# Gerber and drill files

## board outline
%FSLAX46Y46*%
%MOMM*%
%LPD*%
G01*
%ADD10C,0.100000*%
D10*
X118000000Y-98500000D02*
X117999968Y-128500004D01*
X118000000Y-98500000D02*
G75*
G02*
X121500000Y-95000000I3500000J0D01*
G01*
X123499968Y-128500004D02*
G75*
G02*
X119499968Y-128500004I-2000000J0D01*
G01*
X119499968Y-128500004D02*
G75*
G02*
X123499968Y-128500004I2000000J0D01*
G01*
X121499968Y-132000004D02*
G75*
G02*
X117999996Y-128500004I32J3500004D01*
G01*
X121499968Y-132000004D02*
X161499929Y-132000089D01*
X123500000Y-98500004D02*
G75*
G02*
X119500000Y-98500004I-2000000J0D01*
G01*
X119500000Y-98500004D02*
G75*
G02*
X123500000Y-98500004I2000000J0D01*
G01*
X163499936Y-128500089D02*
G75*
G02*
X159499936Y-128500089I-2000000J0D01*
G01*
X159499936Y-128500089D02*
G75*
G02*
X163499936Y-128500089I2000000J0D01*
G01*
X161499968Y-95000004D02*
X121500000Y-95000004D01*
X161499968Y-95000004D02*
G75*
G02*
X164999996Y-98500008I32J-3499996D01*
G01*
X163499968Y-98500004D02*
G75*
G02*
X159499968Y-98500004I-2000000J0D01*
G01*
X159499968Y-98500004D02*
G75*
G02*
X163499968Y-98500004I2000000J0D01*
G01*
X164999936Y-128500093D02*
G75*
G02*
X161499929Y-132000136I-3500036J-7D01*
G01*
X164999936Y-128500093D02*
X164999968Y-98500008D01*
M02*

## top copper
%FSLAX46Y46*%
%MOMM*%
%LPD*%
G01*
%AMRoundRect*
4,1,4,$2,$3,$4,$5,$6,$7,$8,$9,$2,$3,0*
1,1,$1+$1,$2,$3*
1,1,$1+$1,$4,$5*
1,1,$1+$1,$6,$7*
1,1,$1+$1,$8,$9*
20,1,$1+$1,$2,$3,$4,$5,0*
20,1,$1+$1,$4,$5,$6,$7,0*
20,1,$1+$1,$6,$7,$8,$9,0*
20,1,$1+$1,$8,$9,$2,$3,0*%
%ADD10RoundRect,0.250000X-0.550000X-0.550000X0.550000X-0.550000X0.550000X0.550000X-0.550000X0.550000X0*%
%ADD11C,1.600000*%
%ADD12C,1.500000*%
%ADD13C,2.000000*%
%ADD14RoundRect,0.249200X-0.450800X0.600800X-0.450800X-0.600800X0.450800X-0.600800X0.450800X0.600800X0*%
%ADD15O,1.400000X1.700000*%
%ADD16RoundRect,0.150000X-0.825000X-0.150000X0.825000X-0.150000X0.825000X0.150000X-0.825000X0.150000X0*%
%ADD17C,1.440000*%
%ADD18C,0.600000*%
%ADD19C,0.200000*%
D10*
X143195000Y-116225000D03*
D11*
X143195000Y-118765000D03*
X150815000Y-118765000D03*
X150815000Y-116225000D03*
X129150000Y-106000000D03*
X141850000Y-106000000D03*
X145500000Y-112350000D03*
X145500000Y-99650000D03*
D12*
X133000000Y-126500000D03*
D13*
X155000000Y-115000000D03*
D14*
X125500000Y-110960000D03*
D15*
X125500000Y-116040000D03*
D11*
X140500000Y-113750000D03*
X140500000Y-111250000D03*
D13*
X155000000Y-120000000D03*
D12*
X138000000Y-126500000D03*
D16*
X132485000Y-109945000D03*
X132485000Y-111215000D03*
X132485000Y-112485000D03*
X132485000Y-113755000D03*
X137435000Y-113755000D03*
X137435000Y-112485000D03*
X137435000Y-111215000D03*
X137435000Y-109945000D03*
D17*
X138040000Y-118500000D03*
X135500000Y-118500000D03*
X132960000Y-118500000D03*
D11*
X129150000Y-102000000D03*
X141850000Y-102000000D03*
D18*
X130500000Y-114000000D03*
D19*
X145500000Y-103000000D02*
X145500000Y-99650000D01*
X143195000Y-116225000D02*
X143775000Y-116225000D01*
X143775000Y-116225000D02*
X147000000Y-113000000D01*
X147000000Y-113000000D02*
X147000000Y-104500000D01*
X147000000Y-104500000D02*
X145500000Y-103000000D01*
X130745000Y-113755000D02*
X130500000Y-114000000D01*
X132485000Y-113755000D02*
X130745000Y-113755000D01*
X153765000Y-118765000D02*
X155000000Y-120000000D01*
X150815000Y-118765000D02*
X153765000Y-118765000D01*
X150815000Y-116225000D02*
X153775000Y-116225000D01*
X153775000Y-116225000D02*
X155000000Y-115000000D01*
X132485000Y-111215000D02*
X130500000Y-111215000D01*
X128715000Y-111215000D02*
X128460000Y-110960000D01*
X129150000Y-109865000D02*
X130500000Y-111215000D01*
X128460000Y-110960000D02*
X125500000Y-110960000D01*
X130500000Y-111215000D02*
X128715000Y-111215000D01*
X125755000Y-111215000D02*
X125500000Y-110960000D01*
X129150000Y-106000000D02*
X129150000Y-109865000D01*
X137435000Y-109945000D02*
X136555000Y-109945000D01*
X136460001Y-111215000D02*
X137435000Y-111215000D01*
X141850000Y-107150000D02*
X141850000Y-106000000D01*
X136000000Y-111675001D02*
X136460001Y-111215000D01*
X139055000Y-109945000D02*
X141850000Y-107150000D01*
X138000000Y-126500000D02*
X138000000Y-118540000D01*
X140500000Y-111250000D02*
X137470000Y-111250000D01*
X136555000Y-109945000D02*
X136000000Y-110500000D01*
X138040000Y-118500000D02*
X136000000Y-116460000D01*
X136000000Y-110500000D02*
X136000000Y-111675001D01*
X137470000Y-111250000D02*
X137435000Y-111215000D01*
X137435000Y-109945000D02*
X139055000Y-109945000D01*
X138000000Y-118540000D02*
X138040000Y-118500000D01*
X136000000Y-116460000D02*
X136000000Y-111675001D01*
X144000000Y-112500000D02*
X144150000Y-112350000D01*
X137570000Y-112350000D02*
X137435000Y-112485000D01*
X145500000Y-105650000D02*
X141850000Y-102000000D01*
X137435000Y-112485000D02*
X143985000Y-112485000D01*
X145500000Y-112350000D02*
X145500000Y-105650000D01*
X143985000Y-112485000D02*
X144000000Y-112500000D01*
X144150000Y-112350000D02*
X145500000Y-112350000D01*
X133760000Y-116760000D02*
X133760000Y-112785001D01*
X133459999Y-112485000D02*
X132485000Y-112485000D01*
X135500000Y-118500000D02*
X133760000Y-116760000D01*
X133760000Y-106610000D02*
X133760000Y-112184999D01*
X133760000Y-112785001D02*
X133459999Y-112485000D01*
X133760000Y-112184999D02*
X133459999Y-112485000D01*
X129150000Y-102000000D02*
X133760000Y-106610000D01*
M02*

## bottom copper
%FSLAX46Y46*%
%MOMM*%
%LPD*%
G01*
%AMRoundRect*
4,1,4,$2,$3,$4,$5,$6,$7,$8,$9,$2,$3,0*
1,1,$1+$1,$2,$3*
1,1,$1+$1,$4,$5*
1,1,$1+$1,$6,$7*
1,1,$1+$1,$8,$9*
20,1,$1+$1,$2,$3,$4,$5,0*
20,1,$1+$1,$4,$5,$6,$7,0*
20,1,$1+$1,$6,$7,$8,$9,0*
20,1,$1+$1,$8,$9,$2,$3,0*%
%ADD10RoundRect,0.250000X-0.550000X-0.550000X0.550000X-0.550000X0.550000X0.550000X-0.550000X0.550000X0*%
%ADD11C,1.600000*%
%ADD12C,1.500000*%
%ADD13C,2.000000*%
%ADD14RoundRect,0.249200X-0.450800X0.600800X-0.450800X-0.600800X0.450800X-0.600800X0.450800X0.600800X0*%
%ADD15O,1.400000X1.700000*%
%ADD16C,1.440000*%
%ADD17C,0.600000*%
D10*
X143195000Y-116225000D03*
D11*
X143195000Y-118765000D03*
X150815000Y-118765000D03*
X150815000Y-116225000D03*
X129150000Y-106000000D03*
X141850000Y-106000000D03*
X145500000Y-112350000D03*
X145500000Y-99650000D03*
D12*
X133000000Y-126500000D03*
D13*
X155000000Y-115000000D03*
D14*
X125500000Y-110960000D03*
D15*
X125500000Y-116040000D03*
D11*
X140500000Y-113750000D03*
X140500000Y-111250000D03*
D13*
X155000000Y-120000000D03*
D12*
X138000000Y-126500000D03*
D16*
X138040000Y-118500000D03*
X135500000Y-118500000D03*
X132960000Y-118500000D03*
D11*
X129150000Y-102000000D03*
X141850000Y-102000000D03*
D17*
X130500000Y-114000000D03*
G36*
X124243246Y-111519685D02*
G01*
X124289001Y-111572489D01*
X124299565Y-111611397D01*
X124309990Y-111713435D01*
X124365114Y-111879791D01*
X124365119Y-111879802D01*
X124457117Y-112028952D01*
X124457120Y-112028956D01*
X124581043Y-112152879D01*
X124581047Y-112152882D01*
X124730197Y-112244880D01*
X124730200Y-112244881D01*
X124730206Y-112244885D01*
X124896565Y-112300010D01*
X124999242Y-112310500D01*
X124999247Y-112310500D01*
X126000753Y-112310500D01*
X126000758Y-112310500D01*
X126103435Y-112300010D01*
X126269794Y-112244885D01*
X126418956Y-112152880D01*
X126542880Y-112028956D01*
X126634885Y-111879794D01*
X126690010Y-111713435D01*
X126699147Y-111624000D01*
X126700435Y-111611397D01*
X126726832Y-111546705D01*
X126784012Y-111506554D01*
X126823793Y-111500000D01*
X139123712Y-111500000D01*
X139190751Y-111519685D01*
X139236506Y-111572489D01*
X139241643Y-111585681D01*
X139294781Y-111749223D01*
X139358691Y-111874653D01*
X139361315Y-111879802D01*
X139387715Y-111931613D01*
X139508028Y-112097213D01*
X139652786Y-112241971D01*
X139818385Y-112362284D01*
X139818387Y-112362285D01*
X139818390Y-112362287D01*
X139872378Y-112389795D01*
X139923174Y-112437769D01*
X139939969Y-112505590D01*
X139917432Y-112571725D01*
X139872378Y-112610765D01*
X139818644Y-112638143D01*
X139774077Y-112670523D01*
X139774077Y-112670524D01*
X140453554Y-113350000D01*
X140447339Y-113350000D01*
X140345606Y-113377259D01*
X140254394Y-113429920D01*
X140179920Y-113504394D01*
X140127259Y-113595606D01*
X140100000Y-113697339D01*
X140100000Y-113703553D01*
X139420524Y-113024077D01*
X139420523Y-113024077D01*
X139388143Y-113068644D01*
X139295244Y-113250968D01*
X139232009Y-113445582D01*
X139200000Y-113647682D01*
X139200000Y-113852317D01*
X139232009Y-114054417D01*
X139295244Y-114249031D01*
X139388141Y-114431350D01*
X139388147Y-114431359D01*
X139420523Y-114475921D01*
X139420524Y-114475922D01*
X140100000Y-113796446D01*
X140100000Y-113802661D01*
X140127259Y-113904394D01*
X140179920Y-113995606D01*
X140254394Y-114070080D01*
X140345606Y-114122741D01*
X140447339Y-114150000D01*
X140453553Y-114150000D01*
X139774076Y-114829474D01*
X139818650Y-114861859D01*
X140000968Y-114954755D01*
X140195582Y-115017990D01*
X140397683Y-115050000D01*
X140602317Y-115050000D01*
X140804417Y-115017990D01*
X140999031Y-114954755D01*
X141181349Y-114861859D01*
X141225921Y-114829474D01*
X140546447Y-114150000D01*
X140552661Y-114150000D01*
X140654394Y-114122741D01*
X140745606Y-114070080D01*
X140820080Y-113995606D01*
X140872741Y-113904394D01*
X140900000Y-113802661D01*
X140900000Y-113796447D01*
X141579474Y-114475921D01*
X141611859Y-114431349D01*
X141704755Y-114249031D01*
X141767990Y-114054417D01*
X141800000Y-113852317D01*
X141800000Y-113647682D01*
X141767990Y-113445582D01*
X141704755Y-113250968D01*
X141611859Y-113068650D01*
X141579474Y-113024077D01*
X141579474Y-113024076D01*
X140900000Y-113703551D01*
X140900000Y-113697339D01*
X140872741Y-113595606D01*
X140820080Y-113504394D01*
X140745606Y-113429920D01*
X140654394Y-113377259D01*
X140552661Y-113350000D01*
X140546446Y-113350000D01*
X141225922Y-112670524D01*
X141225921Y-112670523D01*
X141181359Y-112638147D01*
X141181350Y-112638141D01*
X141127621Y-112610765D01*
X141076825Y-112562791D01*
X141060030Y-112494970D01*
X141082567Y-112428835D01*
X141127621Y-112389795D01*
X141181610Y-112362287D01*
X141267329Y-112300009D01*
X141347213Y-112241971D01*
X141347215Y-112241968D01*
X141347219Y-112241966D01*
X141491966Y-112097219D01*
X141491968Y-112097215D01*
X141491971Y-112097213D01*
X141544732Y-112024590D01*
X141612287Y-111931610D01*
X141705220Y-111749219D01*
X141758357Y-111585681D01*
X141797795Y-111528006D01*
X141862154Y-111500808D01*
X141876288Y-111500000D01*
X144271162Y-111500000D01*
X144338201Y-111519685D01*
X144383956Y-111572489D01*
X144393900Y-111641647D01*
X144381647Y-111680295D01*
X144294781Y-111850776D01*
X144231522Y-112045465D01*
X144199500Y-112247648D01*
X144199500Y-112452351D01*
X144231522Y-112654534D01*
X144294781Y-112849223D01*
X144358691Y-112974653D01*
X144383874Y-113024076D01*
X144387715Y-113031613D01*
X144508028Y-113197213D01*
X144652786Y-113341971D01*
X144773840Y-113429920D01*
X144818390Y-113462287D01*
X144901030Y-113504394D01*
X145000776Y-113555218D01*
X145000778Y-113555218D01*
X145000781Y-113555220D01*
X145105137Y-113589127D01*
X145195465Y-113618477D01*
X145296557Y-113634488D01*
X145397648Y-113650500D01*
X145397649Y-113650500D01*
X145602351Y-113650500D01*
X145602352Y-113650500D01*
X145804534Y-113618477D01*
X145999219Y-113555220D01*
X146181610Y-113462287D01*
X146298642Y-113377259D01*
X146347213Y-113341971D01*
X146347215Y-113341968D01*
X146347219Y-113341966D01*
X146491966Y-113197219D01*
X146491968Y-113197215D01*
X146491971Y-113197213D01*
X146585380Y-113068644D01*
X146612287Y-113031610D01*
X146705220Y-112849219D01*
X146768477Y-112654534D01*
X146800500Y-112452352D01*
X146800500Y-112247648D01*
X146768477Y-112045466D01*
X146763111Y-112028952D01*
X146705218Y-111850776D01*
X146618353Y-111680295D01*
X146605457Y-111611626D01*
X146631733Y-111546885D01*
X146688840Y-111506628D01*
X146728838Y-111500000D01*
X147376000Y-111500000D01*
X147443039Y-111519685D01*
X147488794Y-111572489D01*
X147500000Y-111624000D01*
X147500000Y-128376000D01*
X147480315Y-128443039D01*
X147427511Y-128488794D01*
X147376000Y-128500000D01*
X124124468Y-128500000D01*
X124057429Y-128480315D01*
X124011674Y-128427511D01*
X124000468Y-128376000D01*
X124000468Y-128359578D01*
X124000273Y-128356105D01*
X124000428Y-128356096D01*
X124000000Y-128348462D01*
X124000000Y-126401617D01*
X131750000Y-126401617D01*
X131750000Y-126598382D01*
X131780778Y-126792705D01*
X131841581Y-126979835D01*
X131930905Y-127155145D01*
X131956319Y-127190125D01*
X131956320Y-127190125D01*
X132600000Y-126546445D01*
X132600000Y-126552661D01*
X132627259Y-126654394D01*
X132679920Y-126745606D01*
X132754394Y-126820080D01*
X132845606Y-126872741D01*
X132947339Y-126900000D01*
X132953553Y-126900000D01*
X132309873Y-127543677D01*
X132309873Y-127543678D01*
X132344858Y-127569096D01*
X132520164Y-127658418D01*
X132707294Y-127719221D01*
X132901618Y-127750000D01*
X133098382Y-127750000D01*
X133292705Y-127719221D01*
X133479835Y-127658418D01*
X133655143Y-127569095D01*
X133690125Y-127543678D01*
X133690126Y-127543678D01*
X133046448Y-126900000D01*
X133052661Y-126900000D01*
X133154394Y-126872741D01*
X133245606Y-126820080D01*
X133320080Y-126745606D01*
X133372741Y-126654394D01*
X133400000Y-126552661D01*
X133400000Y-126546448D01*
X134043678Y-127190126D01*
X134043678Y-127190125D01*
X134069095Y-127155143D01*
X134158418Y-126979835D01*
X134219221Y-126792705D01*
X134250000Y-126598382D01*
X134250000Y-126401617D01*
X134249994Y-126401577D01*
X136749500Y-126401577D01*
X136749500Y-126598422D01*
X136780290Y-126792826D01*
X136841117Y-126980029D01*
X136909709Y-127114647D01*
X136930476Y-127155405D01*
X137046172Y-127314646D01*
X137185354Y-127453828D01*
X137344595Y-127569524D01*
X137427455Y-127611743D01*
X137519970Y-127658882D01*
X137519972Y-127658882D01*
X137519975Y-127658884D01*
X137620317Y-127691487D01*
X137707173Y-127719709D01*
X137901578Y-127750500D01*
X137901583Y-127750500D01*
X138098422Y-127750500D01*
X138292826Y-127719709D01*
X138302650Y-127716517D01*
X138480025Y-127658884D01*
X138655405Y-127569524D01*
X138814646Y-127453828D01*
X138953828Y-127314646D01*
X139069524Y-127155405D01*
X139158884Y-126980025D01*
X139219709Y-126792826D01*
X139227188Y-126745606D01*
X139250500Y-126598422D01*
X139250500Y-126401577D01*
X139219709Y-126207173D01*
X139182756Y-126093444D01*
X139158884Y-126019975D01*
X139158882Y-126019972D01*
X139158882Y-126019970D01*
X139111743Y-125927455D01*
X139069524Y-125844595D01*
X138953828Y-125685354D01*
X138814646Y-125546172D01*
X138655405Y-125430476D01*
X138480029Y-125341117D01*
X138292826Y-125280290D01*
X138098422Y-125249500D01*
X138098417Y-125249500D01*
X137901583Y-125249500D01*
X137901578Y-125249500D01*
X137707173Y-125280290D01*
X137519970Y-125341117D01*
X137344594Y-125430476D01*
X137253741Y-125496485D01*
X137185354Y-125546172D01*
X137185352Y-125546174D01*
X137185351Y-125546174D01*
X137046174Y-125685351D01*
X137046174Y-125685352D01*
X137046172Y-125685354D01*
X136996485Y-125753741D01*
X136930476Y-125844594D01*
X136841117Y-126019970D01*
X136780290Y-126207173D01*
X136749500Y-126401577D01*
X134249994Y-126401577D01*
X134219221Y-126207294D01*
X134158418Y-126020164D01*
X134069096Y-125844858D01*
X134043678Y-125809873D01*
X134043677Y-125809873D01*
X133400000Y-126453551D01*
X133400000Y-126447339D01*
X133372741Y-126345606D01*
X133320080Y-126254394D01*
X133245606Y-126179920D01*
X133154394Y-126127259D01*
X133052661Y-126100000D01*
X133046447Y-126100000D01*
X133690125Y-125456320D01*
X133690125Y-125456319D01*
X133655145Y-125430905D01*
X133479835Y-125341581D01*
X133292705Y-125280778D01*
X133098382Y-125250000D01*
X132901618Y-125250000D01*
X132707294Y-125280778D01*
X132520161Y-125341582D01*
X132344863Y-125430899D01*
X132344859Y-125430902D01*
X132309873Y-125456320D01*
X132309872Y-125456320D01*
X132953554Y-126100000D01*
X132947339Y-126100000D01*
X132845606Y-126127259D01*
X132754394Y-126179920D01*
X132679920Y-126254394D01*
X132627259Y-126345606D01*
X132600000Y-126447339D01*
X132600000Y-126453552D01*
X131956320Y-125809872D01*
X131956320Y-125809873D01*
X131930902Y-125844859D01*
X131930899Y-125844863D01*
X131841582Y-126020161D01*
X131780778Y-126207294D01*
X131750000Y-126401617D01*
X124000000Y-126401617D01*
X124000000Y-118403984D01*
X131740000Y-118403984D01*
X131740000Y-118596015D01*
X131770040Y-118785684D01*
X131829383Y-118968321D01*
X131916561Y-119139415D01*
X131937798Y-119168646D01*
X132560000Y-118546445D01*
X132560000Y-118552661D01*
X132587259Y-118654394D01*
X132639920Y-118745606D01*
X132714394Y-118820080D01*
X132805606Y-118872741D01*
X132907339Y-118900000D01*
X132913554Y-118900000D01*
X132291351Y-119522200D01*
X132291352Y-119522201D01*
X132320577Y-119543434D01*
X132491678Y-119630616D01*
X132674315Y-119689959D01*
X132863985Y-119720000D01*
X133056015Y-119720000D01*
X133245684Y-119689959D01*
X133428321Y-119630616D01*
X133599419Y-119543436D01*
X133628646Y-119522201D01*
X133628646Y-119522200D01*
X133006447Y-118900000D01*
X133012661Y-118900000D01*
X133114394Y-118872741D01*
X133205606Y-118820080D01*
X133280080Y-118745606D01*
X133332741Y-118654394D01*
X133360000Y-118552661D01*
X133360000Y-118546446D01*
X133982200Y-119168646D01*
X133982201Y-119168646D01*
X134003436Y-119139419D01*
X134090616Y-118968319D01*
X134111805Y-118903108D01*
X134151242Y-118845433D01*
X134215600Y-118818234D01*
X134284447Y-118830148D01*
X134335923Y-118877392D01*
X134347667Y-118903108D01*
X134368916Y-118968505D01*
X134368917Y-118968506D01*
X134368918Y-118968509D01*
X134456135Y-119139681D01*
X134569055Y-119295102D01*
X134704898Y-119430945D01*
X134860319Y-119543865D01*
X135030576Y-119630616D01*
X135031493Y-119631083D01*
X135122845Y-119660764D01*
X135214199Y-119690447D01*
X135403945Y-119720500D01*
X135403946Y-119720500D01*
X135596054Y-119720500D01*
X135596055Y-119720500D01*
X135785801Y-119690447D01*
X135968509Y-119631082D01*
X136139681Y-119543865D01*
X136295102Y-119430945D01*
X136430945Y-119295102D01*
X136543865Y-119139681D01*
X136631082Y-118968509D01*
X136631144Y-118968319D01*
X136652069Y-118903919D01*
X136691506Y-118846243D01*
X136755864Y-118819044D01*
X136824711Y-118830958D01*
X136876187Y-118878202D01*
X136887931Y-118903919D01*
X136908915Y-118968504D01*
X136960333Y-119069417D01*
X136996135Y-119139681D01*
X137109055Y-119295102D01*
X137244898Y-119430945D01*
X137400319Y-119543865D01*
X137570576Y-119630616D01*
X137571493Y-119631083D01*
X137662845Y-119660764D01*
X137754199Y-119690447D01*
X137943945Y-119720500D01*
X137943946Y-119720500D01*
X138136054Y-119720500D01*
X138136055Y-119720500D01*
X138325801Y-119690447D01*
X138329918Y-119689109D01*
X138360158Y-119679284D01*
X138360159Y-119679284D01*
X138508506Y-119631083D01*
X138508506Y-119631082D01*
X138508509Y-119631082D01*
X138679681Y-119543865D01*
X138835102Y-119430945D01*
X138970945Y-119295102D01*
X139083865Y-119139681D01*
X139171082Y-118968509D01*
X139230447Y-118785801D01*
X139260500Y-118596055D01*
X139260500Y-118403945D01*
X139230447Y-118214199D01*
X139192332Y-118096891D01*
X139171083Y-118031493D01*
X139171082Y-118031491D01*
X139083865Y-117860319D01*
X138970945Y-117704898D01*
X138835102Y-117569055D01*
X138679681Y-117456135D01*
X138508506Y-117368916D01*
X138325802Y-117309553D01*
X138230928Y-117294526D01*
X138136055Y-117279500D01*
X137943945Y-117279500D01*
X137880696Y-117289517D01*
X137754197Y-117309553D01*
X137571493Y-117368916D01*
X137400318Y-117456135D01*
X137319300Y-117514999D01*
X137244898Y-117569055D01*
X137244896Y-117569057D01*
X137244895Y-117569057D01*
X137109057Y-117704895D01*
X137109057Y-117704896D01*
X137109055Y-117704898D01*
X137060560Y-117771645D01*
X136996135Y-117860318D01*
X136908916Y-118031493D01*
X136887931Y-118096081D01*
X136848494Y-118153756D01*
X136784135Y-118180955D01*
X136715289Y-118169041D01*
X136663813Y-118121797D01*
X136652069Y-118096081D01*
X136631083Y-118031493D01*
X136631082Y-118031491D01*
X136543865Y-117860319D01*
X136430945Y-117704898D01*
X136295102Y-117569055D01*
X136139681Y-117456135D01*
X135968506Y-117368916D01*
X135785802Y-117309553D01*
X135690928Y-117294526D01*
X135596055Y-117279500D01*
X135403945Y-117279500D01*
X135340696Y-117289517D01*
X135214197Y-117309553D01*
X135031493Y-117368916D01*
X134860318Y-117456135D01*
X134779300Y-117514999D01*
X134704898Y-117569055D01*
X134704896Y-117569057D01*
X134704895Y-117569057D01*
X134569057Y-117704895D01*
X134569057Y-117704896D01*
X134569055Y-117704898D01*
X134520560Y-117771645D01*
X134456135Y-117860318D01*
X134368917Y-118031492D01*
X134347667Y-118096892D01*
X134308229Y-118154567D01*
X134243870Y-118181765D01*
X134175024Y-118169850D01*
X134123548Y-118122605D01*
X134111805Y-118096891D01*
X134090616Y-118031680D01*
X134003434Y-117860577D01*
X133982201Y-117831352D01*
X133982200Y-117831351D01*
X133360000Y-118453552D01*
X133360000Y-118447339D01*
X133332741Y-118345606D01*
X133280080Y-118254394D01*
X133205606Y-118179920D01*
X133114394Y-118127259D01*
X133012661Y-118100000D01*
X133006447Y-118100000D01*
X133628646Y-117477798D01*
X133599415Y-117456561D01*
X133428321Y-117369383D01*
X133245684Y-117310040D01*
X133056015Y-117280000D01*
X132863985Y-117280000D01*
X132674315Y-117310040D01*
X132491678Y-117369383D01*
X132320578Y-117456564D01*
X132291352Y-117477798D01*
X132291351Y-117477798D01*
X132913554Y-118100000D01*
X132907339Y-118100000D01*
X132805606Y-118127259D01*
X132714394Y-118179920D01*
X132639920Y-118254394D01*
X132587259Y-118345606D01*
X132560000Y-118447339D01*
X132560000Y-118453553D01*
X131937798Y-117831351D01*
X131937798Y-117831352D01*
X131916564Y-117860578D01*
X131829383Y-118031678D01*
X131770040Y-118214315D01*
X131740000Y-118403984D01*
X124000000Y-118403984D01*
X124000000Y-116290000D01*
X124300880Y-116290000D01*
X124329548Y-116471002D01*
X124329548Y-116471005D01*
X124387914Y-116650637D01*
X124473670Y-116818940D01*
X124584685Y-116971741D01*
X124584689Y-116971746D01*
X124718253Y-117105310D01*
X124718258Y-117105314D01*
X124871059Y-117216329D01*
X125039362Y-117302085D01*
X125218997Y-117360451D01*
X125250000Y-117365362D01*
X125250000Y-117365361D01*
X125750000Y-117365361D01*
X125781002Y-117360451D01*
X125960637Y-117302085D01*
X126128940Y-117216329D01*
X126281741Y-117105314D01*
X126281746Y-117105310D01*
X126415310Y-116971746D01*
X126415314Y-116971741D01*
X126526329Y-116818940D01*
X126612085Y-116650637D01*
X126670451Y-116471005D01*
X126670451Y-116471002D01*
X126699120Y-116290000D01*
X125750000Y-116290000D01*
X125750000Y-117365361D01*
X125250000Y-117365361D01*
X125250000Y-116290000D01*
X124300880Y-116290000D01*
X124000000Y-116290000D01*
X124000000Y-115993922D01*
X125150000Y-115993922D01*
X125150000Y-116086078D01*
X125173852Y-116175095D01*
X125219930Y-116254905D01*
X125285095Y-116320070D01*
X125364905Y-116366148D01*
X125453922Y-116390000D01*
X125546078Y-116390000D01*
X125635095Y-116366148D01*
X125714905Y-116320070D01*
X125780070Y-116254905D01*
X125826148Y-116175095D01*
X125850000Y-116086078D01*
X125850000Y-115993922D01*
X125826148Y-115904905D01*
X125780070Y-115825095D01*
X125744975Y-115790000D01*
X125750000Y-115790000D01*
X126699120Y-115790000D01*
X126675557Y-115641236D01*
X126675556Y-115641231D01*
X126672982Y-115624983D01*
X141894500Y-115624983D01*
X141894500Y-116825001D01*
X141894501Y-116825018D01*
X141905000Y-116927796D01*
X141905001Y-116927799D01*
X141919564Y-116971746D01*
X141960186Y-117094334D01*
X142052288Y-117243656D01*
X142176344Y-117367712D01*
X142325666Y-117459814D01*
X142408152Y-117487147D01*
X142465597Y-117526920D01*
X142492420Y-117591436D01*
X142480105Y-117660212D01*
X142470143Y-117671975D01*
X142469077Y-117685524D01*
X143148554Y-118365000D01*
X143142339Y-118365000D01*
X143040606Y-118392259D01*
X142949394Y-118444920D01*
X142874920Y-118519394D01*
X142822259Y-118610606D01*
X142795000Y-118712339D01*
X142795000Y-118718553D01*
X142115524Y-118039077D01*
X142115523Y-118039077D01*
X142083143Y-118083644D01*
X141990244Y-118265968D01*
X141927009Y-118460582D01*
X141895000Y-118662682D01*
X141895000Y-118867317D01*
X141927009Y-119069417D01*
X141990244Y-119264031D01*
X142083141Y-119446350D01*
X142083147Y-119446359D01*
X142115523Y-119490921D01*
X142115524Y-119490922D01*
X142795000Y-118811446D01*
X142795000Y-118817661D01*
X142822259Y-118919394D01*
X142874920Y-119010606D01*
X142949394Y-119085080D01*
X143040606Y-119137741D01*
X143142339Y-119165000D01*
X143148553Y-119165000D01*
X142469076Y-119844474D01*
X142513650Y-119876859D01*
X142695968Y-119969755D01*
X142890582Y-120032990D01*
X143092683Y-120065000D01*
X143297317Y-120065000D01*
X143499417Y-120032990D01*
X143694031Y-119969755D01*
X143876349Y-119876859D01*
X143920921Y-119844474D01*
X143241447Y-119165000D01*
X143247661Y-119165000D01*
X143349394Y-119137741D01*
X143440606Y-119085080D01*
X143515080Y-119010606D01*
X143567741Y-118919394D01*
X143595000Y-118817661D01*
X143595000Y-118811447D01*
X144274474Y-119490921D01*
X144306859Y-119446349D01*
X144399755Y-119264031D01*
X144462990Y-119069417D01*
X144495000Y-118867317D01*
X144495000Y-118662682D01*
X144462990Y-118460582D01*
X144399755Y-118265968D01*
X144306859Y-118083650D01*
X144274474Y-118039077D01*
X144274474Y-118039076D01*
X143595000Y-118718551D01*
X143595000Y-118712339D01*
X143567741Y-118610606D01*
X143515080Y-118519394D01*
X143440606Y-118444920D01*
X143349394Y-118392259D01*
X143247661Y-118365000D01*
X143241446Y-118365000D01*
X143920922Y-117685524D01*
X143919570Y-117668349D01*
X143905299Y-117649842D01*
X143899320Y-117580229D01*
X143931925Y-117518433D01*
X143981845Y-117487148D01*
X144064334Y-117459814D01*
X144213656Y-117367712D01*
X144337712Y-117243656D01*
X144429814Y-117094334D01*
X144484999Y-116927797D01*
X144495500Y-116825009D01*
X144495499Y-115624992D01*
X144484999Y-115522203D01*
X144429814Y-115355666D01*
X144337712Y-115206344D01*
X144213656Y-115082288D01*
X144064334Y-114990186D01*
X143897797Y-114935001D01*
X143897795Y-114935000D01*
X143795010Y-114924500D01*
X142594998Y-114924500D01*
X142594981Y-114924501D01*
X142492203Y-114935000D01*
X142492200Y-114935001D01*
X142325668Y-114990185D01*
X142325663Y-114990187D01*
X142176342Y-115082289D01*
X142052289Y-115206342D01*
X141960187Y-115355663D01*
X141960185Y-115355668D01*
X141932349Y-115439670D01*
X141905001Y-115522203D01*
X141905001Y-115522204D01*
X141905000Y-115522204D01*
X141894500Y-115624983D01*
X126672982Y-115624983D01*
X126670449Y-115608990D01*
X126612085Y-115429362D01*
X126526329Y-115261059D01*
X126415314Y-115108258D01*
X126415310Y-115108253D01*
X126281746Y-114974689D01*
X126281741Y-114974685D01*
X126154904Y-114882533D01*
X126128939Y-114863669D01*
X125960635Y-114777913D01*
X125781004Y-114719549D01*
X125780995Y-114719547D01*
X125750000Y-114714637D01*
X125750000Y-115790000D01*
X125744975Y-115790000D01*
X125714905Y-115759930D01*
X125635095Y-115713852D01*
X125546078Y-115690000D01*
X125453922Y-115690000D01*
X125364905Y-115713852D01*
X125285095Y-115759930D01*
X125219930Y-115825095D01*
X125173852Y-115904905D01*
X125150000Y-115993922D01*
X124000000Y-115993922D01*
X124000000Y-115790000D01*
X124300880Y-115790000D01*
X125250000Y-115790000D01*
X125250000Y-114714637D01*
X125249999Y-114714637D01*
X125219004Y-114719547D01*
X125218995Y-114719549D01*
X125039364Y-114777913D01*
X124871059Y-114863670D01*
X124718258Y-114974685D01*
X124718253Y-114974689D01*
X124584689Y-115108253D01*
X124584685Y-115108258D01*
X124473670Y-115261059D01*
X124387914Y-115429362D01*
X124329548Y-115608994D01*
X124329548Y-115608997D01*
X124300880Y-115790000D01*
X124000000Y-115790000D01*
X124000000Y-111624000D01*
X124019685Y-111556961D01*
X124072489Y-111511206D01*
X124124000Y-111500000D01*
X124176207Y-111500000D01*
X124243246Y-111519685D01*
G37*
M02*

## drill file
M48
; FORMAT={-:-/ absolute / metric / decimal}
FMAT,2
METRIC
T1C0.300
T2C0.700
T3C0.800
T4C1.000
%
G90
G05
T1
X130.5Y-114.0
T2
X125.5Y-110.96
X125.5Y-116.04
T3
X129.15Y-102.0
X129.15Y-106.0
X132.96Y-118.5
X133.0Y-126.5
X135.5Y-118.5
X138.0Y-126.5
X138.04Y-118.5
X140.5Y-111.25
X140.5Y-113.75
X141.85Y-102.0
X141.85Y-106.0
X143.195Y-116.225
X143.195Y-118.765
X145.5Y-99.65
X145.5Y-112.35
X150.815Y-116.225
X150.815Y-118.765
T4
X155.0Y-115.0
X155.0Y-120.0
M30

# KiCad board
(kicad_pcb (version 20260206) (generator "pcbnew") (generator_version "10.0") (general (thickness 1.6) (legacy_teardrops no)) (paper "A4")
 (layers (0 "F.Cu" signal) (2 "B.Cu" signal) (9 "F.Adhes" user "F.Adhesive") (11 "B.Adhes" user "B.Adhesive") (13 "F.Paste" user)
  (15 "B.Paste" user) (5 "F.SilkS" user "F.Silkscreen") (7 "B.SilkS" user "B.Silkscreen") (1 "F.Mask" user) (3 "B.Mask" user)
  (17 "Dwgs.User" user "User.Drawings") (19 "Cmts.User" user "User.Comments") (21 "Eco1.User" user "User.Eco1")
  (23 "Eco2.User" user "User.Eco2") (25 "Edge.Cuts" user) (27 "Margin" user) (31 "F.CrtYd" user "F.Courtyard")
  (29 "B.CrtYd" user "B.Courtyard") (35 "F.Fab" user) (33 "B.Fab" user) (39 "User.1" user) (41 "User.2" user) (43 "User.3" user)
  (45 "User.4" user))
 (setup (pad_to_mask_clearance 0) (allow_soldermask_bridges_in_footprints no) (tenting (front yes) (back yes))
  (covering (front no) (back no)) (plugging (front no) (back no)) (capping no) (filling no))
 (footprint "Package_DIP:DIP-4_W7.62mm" (layer "F.Cu") (at 143.195 116.225)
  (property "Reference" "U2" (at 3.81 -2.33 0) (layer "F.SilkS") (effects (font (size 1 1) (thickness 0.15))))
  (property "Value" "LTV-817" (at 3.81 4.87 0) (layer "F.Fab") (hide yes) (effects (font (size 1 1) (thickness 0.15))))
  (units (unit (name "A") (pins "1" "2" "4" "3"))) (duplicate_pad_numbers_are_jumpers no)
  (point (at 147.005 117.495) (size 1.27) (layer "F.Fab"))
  (pad "1" thru_hole roundrect (at 0 0) (size 1.6 1.6) (drill 0.8) (layers "*.Cu" "*.Mask") (remove_unused_layers no)
   (roundrect_rratio 0.15625) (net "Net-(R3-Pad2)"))
  (pad "2" thru_hole circle (at 0 2.54) (size 1.6 1.6) (drill 0.8) (layers "*.Cu" "*.Mask") (remove_unused_layers no) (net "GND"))
  (pad "3" thru_hole circle (at 7.62 2.54) (size 1.6 1.6) (drill 0.8) (layers "*.Cu" "*.Mask") (remove_unused_layers no)
   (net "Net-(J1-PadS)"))
  (pad "4" thru_hole circle (at 7.62 0) (size 1.6 1.6) (drill 0.8) (layers "*.Cu" "*.Mask") (remove_unused_layers no) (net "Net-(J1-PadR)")))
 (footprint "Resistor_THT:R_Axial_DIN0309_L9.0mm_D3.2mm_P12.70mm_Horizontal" (layer "F.Cu") (at 129.15 106)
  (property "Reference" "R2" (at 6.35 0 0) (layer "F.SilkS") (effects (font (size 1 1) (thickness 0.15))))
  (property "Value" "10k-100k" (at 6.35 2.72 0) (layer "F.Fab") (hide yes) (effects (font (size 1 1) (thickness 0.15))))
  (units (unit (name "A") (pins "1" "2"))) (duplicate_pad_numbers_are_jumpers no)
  (pad "1" thru_hole circle (at 0 0) (size 1.6 1.6) (drill 0.8) (layers "*.Cu" "*.Mask") (remove_unused_layers no) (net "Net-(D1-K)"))
  (pad "2" thru_hole circle (at 12.7 0) (size 1.6 1.6) (drill 0.8) (layers "*.Cu" "*.Mask") (remove_unused_layers no) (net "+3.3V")))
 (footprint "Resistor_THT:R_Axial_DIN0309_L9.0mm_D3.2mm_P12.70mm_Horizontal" (layer "F.Cu") (at 145.5 112.35 90)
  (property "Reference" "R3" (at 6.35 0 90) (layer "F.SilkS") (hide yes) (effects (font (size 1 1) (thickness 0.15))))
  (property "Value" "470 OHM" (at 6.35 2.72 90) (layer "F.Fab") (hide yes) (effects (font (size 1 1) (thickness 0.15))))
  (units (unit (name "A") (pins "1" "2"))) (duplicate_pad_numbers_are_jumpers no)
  (pad "1" thru_hole circle (at 0 0 90) (size 1.6 1.6) (drill 0.8) (layers "*.Cu" "*.Mask") (remove_unused_layers no) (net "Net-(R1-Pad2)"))
  (pad "2" thru_hole circle (at 12.7 0 90) (size 1.6 1.6) (drill 0.8) (layers "*.Cu" "*.Mask") (remove_unused_layers no)
   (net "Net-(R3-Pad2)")))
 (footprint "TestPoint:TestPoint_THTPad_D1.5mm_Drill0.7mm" (layer "F.Cu") (at 133 126.5 180)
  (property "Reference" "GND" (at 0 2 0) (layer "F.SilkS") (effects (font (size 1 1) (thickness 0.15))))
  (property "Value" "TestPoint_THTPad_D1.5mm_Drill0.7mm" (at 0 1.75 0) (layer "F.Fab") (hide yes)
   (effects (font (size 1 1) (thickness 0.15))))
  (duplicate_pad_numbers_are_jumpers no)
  (pad "1" thru_hole circle (at 0 0 180) (size 1.5 1.5) (drill 0.8) (layers "*.Cu" "*.Mask") (remove_unused_layers no) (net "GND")))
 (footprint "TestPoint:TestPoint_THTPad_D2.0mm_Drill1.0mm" (layer "F.Cu") (at 155 115)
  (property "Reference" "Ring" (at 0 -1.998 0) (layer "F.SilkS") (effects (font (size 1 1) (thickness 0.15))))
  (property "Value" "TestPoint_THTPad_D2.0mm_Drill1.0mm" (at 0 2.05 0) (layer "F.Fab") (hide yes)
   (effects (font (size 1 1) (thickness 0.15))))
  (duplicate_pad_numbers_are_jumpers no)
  (pad "1" thru_hole circle (at 0 0) (size 2 2) (drill 1) (layers "*.Cu" "*.Mask") (remove_unused_layers no) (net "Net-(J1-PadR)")))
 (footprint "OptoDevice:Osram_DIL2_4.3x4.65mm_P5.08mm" (layer "F.Cu") (at 125.5 110.96 -90)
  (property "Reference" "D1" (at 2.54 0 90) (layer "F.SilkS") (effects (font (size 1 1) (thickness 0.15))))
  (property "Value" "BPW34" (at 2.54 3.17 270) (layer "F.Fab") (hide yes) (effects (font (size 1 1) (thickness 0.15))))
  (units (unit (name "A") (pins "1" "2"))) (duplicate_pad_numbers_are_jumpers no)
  (pad "1" thru_hole roundrect (at 0 0 270) (size 1.7 1.4) (drill 0.7) (layers "*.Cu" "*.Mask") (remove_unused_layers no)
   (roundrect_rratio 0.178) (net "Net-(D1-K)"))
  (pad "2" thru_hole oval (at 5.08 0 270) (size 1.7 1.4) (drill 0.7) (layers "*.Cu" "*.Mask") (remove_unused_layers no) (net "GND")))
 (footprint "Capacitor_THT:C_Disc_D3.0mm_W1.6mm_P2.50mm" (layer "F.Cu") (at 140.5 113.75 90)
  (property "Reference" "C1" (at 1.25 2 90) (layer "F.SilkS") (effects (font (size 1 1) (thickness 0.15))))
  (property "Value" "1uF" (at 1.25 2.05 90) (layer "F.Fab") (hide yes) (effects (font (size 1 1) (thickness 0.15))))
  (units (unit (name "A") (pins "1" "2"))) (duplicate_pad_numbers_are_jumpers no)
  (pad "1" thru_hole circle (at 0 0 90) (size 1.6 1.6) (drill 0.8) (layers "*.Cu" "*.Mask") (remove_unused_layers no) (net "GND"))
  (pad "2" thru_hole circle (at 2.5 0 90) (size 1.6 1.6) (drill 0.8) (layers "*.Cu" "*.Mask") (remove_unused_layers no) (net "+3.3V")))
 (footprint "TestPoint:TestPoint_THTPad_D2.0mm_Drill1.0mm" (layer "F.Cu") (at 155 120)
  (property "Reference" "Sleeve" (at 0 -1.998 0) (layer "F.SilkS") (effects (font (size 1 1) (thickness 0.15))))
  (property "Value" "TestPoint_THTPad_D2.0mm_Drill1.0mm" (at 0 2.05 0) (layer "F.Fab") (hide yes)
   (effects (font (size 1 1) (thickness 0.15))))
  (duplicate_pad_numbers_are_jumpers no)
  (pad "1" thru_hole circle (at 0 0) (size 2 2) (drill 1) (layers "*.Cu" "*.Mask") (remove_unused_layers no) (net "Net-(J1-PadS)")))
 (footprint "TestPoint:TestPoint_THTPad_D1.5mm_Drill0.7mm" (layer "F.Cu") (at 138 126.5 180)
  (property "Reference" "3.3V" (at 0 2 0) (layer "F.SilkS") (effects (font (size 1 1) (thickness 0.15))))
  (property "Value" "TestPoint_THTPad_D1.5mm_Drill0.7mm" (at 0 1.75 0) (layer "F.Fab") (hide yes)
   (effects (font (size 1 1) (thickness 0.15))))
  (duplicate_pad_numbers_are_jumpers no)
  (pad "1" thru_hole circle (at 0 0 180) (size 1.5 1.5) (drill 0.8) (layers "*.Cu" "*.Mask") (remove_unused_layers no) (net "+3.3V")))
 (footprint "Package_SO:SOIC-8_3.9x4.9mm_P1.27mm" (layer "F.Cu") (at 134.96 111.85)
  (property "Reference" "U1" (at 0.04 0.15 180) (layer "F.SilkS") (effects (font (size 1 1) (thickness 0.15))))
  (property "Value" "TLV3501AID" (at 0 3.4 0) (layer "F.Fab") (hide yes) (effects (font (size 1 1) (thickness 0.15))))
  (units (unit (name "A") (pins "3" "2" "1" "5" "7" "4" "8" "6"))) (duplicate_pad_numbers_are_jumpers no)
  (pad "1" smd roundrect (at -2.475 -1.905) (size 1.95 0.6) (layers "F.Cu" "F.Mask" "F.Paste") (roundrect_rratio 0.25)
   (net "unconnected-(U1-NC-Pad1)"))
  (pad "2" smd roundrect (at -2.475 -0.635) (size 1.95 0.6) (layers "F.Cu" "F.Mask" "F.Paste") (roundrect_rratio 0.25) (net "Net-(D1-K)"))
  (pad "3" smd roundrect (at -2.475 0.635) (size 1.95 0.6) (layers "F.Cu" "F.Mask" "F.Paste") (roundrect_rratio 0.25) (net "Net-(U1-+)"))
  (pad "4" smd roundrect (at -2.475 1.905) (size 1.95 0.6) (layers "F.Cu" "F.Mask" "F.Paste") (roundrect_rratio 0.25) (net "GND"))
  (pad "5" smd roundrect (at 2.475 1.905) (size 1.95 0.6) (layers "F.Cu" "F.Mask" "F.Paste") (roundrect_rratio 0.25)
   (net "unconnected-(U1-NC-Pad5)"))
  (pad "6" smd roundrect (at 2.475 0.635) (size 1.95 0.6) (layers "F.Cu" "F.Mask" "F.Paste") (roundrect_rratio 0.25) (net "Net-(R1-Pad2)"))
  (pad "7" smd roundrect (at 2.475 -0.635) (size 1.95 0.6) (layers "F.Cu" "F.Mask" "F.Paste") (roundrect_rratio 0.25) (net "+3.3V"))
  (pad "8" smd roundrect (at 2.475 -1.905) (size 1.95 0.6) (layers "F.Cu" "F.Mask" "F.Paste") (roundrect_rratio 0.25) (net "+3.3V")))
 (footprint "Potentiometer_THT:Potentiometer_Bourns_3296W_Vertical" (layer "F.Cu") (at 138.04 118.5)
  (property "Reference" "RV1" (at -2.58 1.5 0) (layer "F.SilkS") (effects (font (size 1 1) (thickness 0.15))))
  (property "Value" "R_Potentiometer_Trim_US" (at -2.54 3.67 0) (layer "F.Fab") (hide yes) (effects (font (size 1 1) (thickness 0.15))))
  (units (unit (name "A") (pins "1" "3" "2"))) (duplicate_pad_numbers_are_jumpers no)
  (pad "1" thru_hole circle (at 0 0) (size 1.44 1.44) (drill 0.8) (layers "*.Cu" "*.Mask") (remove_unused_layers no) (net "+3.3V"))
  (pad "2" thru_hole circle (at -2.54 0) (size 1.44 1.44) (drill 0.8) (layers "*.Cu" "*.Mask") (remove_unused_layers no) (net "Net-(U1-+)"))
  (pad "3" thru_hole circle (at -5.08 0) (size 1.44 1.44) (drill 0.8) (layers "*.Cu" "*.Mask") (remove_unused_layers no) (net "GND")))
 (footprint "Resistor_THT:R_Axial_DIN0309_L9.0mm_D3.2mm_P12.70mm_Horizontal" (layer "F.Cu") (at 129.15 102)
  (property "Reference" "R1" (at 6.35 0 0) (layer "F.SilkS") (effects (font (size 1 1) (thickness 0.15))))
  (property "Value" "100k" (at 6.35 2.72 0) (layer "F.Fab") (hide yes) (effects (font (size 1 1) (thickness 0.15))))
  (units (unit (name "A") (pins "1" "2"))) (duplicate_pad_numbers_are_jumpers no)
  (pad "1" thru_hole circle (at 0 0) (size 1.6 1.6) (drill 0.8) (layers "*.Cu" "*.Mask") (remove_unused_layers no) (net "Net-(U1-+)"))
  (pad "2" thru_hole circle (at 12.7 0) (size 1.6 1.6) (drill 0.8) (layers "*.Cu" "*.Mask") (remove_unused_layers no) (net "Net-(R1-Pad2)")))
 (gr_line (start 118 98.5) (end 117.999968 128.500004) (stroke (width 0.1) (type default)) (layer "Edge.Cuts"))
 (gr_arc (start 118 98.5) (mid 119.025128 96.02513) (end 121.5 95.000004) (stroke (width 0.1) (type default)) (layer "Edge.Cuts"))
 (gr_circle (center 121.499968 128.500004) (end 121.499968 126.500004) (stroke (width 0.1) (type default)) (fill no) (layer "Edge.Cuts"))
 (gr_arc (start 121.499968 132.000004) (mid 119.025094 130.974878) (end 117.999968 128.500004) (stroke (width 0.1) (type default))
  (layer "Edge.Cuts"))
 (gr_line (start 121.499968 132.000004) (end 161.499929 132.000089) (stroke (width 0.1) (type default)) (layer "Edge.Cuts"))
 (gr_circle (center 121.5 98.500004) (end 121.5 96.500004) (stroke (width 0.1) (type default)) (fill no) (layer "Edge.Cuts"))
 (gr_circle (center 161.499936 128.500089) (end 161.499936 126.500089) (stroke (width 0.1) (type default)) (fill no) (layer "Edge.Cuts"))
 (gr_line (start 161.499968 95.000004) (end 121.5 95.000004) (stroke (width 0.1) (type default)) (layer "Edge.Cuts"))
 (gr_arc (start 161.499968 95.000004) (mid 163.974843 96.025132) (end 164.999968 98.500008) (stroke (width 0.1) (type default))
  (layer "Edge.Cuts"))
 (gr_circle (center 161.499968 98.500004) (end 161.499968 96.500004) (stroke (width 0.1) (type default)) (fill no) (layer "Edge.Cuts"))
 (gr_arc (start 164.999936 128.500093) (mid 163.974806 130.974967) (end 161.499929 132.000089) (stroke (width 0.1) (type default))
  (layer "Edge.Cuts"))
 (gr_line (start 164.999936 128.500093) (end 164.999968 98.500008) (stroke (width 0.1) (type default)) (layer "Edge.Cuts"))
 (segment (start 145.5 103) (end 145.5 99.65) (width 0.2) (layer "F.Cu") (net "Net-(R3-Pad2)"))
 (segment (start 143.195 116.225) (end 143.775 116.225) (width 0.2) (layer "F.Cu") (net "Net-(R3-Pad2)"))
 (segment (start 143.775 116.225) (end 147 113) (width 0.2) (layer "F.Cu") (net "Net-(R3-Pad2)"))
 (segment (start 147 113) (end 147 104.5) (width 0.2) (layer "F.Cu") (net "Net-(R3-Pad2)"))
 (segment (start 147 104.5) (end 145.5 103) (width 0.2) (layer "F.Cu") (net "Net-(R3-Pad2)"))
 (segment (start 130.745 113.755) (end 130.5 114) (width 0.2) (layer "F.Cu") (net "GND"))
 (segment (start 132.485 113.755) (end 130.745 113.755) (width 0.2) (layer "F.Cu") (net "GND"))
 (via (at 130.5 114) (size 0.6) (drill 0.3) (layers "F.Cu" "B.Cu") (free yes) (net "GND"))
 (segment (start 153.765 118.765) (end 155 120) (width 0.2) (layer "F.Cu") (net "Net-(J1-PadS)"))
 (segment (start 150.815 118.765) (end 153.765 118.765) (width 0.2) (layer "F.Cu") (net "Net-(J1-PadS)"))
 (segment (start 150.815 116.225) (end 153.775 116.225) (width 0.2) (layer "F.Cu") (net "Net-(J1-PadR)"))
 (segment (start 153.775 116.225) (end 155 115) (width 0.2) (layer "F.Cu") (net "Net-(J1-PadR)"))
 (segment (start 132.485 111.215) (end 130.5 111.215) (width 0.2) (layer "F.Cu") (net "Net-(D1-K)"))
 (segment (start 128.715 111.215) (end 128.46 110.96) (width 0.2) (layer "F.Cu") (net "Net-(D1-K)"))
 (segment (start 129.15 109.865) (end 130.5 111.215) (width 0.2) (layer "F.Cu") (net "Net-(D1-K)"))
 (segment (start 128.46 110.96) (end 125.5 110.96) (width 0.2) (layer "F.Cu") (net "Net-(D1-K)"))
 (segment (start 130.5 111.215) (end 128.715 111.215) (width 0.2) (layer "F.Cu") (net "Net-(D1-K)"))
 (segment (start 125.755 111.215) (end 125.5 110.96) (width 0.2) (layer "F.Cu") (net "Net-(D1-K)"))
 (segment (start 129.15 106) (end 129.15 109.865) (width 0.2) (layer "F.Cu") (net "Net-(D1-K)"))
 (segment (start 137.435 109.945) (end 136.555 109.945) (width 0.2) (layer "F.Cu") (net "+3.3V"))
 (segment (start 136.460001 111.215) (end 137.435 111.215) (width 0.2) (layer "F.Cu") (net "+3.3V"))
 (segment (start 141.85 107.15) (end 141.85 106) (width 0.2) (layer "F.Cu") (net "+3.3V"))
 (segment (start 136 111.675001) (end 136.460001 111.215) (width 0.2) (layer "F.Cu") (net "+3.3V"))
 (segment (start 139.055 109.945) (end 141.85 107.15) (width 0.2) (layer "F.Cu") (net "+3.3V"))
 (segment (start 138 126.5) (end 138 118.54) (width 0.2) (layer "F.Cu") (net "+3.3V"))
 (segment (start 140.5 111.25) (end 137.47 111.25) (width 0.2) (layer "F.Cu") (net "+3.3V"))
 (segment (start 136.555 109.945) (end 136 110.5) (width 0.2) (layer "F.Cu") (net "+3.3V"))
 (segment (start 138.04 118.5) (end 136 116.46) (width 0.2) (layer "F.Cu") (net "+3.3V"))
 (segment (start 136 110.5) (end 136 111.675001) (width 0.2) (layer "F.Cu") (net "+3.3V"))
 (segment (start 137.47 111.25) (end 137.435 111.215) (width 0.2) (layer "F.Cu") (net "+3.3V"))
 (segment (start 137.435 109.945) (end 139.055 109.945) (width 0.2) (layer "F.Cu") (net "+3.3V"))
 (segment (start 138 118.54) (end 138.04 118.5) (width 0.2) (layer "F.Cu") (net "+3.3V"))
 (segment (start 136 116.46) (end 136 111.675001) (width 0.2) (layer "F.Cu") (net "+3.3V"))
 (segment (start 144 112.5) (end 144.15 112.35) (width 0.2) (layer "F.Cu") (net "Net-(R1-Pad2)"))
 (segment (start 137.57 112.35) (end 137.435 112.485) (width 0.2) (layer "F.Cu") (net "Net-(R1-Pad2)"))
 (segment (start 145.5 105.65) (end 141.85 102) (width 0.2) (layer "F.Cu") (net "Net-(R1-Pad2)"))
 (segment (start 137.435 112.485) (end 143.985 112.485) (width 0.2) (layer "F.Cu") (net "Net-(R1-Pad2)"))
 (segment (start 145.5 112.35) (end 145.5 105.65) (width 0.2) (layer "F.Cu") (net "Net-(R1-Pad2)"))
 (segment (start 143.985 112.485) (end 144 112.5) (width 0.2) (layer "F.Cu") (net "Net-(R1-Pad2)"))
 (segment (start 144.15 112.35) (end 145.5 112.35) (width 0.2) (layer "F.Cu") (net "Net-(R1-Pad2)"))
 (segment (start 133.76 116.76) (end 133.76 112.785001) (width 0.2) (layer "F.Cu") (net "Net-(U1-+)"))
 (segment (start 133.459999 112.485) (end 132.485 112.485) (width 0.2) (layer "F.Cu") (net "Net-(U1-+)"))
 (segment (start 135.5 118.5) (end 133.76 116.76) (width 0.2) (layer "F.Cu") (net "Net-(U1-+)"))
 (segment (start 133.76 106.61) (end 133.76 112.184999) (width 0.2) (layer "F.Cu") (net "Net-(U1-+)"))
 (segment (start 133.76 112.785001) (end 133.459999 112.485) (width 0.2) (layer "F.Cu") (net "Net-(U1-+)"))
 (segment (start 133.76 112.184999) (end 133.459999 112.485) (width 0.2) (layer "F.Cu") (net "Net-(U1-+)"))
 (segment (start 129.15 102) (end 133.76 106.61) (width 0.2) (layer "F.Cu") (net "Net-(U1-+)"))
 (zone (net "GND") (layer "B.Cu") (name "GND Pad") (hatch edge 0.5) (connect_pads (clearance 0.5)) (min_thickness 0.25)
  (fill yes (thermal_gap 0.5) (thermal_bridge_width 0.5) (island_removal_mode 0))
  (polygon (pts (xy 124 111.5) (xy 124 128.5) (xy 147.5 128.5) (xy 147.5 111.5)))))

